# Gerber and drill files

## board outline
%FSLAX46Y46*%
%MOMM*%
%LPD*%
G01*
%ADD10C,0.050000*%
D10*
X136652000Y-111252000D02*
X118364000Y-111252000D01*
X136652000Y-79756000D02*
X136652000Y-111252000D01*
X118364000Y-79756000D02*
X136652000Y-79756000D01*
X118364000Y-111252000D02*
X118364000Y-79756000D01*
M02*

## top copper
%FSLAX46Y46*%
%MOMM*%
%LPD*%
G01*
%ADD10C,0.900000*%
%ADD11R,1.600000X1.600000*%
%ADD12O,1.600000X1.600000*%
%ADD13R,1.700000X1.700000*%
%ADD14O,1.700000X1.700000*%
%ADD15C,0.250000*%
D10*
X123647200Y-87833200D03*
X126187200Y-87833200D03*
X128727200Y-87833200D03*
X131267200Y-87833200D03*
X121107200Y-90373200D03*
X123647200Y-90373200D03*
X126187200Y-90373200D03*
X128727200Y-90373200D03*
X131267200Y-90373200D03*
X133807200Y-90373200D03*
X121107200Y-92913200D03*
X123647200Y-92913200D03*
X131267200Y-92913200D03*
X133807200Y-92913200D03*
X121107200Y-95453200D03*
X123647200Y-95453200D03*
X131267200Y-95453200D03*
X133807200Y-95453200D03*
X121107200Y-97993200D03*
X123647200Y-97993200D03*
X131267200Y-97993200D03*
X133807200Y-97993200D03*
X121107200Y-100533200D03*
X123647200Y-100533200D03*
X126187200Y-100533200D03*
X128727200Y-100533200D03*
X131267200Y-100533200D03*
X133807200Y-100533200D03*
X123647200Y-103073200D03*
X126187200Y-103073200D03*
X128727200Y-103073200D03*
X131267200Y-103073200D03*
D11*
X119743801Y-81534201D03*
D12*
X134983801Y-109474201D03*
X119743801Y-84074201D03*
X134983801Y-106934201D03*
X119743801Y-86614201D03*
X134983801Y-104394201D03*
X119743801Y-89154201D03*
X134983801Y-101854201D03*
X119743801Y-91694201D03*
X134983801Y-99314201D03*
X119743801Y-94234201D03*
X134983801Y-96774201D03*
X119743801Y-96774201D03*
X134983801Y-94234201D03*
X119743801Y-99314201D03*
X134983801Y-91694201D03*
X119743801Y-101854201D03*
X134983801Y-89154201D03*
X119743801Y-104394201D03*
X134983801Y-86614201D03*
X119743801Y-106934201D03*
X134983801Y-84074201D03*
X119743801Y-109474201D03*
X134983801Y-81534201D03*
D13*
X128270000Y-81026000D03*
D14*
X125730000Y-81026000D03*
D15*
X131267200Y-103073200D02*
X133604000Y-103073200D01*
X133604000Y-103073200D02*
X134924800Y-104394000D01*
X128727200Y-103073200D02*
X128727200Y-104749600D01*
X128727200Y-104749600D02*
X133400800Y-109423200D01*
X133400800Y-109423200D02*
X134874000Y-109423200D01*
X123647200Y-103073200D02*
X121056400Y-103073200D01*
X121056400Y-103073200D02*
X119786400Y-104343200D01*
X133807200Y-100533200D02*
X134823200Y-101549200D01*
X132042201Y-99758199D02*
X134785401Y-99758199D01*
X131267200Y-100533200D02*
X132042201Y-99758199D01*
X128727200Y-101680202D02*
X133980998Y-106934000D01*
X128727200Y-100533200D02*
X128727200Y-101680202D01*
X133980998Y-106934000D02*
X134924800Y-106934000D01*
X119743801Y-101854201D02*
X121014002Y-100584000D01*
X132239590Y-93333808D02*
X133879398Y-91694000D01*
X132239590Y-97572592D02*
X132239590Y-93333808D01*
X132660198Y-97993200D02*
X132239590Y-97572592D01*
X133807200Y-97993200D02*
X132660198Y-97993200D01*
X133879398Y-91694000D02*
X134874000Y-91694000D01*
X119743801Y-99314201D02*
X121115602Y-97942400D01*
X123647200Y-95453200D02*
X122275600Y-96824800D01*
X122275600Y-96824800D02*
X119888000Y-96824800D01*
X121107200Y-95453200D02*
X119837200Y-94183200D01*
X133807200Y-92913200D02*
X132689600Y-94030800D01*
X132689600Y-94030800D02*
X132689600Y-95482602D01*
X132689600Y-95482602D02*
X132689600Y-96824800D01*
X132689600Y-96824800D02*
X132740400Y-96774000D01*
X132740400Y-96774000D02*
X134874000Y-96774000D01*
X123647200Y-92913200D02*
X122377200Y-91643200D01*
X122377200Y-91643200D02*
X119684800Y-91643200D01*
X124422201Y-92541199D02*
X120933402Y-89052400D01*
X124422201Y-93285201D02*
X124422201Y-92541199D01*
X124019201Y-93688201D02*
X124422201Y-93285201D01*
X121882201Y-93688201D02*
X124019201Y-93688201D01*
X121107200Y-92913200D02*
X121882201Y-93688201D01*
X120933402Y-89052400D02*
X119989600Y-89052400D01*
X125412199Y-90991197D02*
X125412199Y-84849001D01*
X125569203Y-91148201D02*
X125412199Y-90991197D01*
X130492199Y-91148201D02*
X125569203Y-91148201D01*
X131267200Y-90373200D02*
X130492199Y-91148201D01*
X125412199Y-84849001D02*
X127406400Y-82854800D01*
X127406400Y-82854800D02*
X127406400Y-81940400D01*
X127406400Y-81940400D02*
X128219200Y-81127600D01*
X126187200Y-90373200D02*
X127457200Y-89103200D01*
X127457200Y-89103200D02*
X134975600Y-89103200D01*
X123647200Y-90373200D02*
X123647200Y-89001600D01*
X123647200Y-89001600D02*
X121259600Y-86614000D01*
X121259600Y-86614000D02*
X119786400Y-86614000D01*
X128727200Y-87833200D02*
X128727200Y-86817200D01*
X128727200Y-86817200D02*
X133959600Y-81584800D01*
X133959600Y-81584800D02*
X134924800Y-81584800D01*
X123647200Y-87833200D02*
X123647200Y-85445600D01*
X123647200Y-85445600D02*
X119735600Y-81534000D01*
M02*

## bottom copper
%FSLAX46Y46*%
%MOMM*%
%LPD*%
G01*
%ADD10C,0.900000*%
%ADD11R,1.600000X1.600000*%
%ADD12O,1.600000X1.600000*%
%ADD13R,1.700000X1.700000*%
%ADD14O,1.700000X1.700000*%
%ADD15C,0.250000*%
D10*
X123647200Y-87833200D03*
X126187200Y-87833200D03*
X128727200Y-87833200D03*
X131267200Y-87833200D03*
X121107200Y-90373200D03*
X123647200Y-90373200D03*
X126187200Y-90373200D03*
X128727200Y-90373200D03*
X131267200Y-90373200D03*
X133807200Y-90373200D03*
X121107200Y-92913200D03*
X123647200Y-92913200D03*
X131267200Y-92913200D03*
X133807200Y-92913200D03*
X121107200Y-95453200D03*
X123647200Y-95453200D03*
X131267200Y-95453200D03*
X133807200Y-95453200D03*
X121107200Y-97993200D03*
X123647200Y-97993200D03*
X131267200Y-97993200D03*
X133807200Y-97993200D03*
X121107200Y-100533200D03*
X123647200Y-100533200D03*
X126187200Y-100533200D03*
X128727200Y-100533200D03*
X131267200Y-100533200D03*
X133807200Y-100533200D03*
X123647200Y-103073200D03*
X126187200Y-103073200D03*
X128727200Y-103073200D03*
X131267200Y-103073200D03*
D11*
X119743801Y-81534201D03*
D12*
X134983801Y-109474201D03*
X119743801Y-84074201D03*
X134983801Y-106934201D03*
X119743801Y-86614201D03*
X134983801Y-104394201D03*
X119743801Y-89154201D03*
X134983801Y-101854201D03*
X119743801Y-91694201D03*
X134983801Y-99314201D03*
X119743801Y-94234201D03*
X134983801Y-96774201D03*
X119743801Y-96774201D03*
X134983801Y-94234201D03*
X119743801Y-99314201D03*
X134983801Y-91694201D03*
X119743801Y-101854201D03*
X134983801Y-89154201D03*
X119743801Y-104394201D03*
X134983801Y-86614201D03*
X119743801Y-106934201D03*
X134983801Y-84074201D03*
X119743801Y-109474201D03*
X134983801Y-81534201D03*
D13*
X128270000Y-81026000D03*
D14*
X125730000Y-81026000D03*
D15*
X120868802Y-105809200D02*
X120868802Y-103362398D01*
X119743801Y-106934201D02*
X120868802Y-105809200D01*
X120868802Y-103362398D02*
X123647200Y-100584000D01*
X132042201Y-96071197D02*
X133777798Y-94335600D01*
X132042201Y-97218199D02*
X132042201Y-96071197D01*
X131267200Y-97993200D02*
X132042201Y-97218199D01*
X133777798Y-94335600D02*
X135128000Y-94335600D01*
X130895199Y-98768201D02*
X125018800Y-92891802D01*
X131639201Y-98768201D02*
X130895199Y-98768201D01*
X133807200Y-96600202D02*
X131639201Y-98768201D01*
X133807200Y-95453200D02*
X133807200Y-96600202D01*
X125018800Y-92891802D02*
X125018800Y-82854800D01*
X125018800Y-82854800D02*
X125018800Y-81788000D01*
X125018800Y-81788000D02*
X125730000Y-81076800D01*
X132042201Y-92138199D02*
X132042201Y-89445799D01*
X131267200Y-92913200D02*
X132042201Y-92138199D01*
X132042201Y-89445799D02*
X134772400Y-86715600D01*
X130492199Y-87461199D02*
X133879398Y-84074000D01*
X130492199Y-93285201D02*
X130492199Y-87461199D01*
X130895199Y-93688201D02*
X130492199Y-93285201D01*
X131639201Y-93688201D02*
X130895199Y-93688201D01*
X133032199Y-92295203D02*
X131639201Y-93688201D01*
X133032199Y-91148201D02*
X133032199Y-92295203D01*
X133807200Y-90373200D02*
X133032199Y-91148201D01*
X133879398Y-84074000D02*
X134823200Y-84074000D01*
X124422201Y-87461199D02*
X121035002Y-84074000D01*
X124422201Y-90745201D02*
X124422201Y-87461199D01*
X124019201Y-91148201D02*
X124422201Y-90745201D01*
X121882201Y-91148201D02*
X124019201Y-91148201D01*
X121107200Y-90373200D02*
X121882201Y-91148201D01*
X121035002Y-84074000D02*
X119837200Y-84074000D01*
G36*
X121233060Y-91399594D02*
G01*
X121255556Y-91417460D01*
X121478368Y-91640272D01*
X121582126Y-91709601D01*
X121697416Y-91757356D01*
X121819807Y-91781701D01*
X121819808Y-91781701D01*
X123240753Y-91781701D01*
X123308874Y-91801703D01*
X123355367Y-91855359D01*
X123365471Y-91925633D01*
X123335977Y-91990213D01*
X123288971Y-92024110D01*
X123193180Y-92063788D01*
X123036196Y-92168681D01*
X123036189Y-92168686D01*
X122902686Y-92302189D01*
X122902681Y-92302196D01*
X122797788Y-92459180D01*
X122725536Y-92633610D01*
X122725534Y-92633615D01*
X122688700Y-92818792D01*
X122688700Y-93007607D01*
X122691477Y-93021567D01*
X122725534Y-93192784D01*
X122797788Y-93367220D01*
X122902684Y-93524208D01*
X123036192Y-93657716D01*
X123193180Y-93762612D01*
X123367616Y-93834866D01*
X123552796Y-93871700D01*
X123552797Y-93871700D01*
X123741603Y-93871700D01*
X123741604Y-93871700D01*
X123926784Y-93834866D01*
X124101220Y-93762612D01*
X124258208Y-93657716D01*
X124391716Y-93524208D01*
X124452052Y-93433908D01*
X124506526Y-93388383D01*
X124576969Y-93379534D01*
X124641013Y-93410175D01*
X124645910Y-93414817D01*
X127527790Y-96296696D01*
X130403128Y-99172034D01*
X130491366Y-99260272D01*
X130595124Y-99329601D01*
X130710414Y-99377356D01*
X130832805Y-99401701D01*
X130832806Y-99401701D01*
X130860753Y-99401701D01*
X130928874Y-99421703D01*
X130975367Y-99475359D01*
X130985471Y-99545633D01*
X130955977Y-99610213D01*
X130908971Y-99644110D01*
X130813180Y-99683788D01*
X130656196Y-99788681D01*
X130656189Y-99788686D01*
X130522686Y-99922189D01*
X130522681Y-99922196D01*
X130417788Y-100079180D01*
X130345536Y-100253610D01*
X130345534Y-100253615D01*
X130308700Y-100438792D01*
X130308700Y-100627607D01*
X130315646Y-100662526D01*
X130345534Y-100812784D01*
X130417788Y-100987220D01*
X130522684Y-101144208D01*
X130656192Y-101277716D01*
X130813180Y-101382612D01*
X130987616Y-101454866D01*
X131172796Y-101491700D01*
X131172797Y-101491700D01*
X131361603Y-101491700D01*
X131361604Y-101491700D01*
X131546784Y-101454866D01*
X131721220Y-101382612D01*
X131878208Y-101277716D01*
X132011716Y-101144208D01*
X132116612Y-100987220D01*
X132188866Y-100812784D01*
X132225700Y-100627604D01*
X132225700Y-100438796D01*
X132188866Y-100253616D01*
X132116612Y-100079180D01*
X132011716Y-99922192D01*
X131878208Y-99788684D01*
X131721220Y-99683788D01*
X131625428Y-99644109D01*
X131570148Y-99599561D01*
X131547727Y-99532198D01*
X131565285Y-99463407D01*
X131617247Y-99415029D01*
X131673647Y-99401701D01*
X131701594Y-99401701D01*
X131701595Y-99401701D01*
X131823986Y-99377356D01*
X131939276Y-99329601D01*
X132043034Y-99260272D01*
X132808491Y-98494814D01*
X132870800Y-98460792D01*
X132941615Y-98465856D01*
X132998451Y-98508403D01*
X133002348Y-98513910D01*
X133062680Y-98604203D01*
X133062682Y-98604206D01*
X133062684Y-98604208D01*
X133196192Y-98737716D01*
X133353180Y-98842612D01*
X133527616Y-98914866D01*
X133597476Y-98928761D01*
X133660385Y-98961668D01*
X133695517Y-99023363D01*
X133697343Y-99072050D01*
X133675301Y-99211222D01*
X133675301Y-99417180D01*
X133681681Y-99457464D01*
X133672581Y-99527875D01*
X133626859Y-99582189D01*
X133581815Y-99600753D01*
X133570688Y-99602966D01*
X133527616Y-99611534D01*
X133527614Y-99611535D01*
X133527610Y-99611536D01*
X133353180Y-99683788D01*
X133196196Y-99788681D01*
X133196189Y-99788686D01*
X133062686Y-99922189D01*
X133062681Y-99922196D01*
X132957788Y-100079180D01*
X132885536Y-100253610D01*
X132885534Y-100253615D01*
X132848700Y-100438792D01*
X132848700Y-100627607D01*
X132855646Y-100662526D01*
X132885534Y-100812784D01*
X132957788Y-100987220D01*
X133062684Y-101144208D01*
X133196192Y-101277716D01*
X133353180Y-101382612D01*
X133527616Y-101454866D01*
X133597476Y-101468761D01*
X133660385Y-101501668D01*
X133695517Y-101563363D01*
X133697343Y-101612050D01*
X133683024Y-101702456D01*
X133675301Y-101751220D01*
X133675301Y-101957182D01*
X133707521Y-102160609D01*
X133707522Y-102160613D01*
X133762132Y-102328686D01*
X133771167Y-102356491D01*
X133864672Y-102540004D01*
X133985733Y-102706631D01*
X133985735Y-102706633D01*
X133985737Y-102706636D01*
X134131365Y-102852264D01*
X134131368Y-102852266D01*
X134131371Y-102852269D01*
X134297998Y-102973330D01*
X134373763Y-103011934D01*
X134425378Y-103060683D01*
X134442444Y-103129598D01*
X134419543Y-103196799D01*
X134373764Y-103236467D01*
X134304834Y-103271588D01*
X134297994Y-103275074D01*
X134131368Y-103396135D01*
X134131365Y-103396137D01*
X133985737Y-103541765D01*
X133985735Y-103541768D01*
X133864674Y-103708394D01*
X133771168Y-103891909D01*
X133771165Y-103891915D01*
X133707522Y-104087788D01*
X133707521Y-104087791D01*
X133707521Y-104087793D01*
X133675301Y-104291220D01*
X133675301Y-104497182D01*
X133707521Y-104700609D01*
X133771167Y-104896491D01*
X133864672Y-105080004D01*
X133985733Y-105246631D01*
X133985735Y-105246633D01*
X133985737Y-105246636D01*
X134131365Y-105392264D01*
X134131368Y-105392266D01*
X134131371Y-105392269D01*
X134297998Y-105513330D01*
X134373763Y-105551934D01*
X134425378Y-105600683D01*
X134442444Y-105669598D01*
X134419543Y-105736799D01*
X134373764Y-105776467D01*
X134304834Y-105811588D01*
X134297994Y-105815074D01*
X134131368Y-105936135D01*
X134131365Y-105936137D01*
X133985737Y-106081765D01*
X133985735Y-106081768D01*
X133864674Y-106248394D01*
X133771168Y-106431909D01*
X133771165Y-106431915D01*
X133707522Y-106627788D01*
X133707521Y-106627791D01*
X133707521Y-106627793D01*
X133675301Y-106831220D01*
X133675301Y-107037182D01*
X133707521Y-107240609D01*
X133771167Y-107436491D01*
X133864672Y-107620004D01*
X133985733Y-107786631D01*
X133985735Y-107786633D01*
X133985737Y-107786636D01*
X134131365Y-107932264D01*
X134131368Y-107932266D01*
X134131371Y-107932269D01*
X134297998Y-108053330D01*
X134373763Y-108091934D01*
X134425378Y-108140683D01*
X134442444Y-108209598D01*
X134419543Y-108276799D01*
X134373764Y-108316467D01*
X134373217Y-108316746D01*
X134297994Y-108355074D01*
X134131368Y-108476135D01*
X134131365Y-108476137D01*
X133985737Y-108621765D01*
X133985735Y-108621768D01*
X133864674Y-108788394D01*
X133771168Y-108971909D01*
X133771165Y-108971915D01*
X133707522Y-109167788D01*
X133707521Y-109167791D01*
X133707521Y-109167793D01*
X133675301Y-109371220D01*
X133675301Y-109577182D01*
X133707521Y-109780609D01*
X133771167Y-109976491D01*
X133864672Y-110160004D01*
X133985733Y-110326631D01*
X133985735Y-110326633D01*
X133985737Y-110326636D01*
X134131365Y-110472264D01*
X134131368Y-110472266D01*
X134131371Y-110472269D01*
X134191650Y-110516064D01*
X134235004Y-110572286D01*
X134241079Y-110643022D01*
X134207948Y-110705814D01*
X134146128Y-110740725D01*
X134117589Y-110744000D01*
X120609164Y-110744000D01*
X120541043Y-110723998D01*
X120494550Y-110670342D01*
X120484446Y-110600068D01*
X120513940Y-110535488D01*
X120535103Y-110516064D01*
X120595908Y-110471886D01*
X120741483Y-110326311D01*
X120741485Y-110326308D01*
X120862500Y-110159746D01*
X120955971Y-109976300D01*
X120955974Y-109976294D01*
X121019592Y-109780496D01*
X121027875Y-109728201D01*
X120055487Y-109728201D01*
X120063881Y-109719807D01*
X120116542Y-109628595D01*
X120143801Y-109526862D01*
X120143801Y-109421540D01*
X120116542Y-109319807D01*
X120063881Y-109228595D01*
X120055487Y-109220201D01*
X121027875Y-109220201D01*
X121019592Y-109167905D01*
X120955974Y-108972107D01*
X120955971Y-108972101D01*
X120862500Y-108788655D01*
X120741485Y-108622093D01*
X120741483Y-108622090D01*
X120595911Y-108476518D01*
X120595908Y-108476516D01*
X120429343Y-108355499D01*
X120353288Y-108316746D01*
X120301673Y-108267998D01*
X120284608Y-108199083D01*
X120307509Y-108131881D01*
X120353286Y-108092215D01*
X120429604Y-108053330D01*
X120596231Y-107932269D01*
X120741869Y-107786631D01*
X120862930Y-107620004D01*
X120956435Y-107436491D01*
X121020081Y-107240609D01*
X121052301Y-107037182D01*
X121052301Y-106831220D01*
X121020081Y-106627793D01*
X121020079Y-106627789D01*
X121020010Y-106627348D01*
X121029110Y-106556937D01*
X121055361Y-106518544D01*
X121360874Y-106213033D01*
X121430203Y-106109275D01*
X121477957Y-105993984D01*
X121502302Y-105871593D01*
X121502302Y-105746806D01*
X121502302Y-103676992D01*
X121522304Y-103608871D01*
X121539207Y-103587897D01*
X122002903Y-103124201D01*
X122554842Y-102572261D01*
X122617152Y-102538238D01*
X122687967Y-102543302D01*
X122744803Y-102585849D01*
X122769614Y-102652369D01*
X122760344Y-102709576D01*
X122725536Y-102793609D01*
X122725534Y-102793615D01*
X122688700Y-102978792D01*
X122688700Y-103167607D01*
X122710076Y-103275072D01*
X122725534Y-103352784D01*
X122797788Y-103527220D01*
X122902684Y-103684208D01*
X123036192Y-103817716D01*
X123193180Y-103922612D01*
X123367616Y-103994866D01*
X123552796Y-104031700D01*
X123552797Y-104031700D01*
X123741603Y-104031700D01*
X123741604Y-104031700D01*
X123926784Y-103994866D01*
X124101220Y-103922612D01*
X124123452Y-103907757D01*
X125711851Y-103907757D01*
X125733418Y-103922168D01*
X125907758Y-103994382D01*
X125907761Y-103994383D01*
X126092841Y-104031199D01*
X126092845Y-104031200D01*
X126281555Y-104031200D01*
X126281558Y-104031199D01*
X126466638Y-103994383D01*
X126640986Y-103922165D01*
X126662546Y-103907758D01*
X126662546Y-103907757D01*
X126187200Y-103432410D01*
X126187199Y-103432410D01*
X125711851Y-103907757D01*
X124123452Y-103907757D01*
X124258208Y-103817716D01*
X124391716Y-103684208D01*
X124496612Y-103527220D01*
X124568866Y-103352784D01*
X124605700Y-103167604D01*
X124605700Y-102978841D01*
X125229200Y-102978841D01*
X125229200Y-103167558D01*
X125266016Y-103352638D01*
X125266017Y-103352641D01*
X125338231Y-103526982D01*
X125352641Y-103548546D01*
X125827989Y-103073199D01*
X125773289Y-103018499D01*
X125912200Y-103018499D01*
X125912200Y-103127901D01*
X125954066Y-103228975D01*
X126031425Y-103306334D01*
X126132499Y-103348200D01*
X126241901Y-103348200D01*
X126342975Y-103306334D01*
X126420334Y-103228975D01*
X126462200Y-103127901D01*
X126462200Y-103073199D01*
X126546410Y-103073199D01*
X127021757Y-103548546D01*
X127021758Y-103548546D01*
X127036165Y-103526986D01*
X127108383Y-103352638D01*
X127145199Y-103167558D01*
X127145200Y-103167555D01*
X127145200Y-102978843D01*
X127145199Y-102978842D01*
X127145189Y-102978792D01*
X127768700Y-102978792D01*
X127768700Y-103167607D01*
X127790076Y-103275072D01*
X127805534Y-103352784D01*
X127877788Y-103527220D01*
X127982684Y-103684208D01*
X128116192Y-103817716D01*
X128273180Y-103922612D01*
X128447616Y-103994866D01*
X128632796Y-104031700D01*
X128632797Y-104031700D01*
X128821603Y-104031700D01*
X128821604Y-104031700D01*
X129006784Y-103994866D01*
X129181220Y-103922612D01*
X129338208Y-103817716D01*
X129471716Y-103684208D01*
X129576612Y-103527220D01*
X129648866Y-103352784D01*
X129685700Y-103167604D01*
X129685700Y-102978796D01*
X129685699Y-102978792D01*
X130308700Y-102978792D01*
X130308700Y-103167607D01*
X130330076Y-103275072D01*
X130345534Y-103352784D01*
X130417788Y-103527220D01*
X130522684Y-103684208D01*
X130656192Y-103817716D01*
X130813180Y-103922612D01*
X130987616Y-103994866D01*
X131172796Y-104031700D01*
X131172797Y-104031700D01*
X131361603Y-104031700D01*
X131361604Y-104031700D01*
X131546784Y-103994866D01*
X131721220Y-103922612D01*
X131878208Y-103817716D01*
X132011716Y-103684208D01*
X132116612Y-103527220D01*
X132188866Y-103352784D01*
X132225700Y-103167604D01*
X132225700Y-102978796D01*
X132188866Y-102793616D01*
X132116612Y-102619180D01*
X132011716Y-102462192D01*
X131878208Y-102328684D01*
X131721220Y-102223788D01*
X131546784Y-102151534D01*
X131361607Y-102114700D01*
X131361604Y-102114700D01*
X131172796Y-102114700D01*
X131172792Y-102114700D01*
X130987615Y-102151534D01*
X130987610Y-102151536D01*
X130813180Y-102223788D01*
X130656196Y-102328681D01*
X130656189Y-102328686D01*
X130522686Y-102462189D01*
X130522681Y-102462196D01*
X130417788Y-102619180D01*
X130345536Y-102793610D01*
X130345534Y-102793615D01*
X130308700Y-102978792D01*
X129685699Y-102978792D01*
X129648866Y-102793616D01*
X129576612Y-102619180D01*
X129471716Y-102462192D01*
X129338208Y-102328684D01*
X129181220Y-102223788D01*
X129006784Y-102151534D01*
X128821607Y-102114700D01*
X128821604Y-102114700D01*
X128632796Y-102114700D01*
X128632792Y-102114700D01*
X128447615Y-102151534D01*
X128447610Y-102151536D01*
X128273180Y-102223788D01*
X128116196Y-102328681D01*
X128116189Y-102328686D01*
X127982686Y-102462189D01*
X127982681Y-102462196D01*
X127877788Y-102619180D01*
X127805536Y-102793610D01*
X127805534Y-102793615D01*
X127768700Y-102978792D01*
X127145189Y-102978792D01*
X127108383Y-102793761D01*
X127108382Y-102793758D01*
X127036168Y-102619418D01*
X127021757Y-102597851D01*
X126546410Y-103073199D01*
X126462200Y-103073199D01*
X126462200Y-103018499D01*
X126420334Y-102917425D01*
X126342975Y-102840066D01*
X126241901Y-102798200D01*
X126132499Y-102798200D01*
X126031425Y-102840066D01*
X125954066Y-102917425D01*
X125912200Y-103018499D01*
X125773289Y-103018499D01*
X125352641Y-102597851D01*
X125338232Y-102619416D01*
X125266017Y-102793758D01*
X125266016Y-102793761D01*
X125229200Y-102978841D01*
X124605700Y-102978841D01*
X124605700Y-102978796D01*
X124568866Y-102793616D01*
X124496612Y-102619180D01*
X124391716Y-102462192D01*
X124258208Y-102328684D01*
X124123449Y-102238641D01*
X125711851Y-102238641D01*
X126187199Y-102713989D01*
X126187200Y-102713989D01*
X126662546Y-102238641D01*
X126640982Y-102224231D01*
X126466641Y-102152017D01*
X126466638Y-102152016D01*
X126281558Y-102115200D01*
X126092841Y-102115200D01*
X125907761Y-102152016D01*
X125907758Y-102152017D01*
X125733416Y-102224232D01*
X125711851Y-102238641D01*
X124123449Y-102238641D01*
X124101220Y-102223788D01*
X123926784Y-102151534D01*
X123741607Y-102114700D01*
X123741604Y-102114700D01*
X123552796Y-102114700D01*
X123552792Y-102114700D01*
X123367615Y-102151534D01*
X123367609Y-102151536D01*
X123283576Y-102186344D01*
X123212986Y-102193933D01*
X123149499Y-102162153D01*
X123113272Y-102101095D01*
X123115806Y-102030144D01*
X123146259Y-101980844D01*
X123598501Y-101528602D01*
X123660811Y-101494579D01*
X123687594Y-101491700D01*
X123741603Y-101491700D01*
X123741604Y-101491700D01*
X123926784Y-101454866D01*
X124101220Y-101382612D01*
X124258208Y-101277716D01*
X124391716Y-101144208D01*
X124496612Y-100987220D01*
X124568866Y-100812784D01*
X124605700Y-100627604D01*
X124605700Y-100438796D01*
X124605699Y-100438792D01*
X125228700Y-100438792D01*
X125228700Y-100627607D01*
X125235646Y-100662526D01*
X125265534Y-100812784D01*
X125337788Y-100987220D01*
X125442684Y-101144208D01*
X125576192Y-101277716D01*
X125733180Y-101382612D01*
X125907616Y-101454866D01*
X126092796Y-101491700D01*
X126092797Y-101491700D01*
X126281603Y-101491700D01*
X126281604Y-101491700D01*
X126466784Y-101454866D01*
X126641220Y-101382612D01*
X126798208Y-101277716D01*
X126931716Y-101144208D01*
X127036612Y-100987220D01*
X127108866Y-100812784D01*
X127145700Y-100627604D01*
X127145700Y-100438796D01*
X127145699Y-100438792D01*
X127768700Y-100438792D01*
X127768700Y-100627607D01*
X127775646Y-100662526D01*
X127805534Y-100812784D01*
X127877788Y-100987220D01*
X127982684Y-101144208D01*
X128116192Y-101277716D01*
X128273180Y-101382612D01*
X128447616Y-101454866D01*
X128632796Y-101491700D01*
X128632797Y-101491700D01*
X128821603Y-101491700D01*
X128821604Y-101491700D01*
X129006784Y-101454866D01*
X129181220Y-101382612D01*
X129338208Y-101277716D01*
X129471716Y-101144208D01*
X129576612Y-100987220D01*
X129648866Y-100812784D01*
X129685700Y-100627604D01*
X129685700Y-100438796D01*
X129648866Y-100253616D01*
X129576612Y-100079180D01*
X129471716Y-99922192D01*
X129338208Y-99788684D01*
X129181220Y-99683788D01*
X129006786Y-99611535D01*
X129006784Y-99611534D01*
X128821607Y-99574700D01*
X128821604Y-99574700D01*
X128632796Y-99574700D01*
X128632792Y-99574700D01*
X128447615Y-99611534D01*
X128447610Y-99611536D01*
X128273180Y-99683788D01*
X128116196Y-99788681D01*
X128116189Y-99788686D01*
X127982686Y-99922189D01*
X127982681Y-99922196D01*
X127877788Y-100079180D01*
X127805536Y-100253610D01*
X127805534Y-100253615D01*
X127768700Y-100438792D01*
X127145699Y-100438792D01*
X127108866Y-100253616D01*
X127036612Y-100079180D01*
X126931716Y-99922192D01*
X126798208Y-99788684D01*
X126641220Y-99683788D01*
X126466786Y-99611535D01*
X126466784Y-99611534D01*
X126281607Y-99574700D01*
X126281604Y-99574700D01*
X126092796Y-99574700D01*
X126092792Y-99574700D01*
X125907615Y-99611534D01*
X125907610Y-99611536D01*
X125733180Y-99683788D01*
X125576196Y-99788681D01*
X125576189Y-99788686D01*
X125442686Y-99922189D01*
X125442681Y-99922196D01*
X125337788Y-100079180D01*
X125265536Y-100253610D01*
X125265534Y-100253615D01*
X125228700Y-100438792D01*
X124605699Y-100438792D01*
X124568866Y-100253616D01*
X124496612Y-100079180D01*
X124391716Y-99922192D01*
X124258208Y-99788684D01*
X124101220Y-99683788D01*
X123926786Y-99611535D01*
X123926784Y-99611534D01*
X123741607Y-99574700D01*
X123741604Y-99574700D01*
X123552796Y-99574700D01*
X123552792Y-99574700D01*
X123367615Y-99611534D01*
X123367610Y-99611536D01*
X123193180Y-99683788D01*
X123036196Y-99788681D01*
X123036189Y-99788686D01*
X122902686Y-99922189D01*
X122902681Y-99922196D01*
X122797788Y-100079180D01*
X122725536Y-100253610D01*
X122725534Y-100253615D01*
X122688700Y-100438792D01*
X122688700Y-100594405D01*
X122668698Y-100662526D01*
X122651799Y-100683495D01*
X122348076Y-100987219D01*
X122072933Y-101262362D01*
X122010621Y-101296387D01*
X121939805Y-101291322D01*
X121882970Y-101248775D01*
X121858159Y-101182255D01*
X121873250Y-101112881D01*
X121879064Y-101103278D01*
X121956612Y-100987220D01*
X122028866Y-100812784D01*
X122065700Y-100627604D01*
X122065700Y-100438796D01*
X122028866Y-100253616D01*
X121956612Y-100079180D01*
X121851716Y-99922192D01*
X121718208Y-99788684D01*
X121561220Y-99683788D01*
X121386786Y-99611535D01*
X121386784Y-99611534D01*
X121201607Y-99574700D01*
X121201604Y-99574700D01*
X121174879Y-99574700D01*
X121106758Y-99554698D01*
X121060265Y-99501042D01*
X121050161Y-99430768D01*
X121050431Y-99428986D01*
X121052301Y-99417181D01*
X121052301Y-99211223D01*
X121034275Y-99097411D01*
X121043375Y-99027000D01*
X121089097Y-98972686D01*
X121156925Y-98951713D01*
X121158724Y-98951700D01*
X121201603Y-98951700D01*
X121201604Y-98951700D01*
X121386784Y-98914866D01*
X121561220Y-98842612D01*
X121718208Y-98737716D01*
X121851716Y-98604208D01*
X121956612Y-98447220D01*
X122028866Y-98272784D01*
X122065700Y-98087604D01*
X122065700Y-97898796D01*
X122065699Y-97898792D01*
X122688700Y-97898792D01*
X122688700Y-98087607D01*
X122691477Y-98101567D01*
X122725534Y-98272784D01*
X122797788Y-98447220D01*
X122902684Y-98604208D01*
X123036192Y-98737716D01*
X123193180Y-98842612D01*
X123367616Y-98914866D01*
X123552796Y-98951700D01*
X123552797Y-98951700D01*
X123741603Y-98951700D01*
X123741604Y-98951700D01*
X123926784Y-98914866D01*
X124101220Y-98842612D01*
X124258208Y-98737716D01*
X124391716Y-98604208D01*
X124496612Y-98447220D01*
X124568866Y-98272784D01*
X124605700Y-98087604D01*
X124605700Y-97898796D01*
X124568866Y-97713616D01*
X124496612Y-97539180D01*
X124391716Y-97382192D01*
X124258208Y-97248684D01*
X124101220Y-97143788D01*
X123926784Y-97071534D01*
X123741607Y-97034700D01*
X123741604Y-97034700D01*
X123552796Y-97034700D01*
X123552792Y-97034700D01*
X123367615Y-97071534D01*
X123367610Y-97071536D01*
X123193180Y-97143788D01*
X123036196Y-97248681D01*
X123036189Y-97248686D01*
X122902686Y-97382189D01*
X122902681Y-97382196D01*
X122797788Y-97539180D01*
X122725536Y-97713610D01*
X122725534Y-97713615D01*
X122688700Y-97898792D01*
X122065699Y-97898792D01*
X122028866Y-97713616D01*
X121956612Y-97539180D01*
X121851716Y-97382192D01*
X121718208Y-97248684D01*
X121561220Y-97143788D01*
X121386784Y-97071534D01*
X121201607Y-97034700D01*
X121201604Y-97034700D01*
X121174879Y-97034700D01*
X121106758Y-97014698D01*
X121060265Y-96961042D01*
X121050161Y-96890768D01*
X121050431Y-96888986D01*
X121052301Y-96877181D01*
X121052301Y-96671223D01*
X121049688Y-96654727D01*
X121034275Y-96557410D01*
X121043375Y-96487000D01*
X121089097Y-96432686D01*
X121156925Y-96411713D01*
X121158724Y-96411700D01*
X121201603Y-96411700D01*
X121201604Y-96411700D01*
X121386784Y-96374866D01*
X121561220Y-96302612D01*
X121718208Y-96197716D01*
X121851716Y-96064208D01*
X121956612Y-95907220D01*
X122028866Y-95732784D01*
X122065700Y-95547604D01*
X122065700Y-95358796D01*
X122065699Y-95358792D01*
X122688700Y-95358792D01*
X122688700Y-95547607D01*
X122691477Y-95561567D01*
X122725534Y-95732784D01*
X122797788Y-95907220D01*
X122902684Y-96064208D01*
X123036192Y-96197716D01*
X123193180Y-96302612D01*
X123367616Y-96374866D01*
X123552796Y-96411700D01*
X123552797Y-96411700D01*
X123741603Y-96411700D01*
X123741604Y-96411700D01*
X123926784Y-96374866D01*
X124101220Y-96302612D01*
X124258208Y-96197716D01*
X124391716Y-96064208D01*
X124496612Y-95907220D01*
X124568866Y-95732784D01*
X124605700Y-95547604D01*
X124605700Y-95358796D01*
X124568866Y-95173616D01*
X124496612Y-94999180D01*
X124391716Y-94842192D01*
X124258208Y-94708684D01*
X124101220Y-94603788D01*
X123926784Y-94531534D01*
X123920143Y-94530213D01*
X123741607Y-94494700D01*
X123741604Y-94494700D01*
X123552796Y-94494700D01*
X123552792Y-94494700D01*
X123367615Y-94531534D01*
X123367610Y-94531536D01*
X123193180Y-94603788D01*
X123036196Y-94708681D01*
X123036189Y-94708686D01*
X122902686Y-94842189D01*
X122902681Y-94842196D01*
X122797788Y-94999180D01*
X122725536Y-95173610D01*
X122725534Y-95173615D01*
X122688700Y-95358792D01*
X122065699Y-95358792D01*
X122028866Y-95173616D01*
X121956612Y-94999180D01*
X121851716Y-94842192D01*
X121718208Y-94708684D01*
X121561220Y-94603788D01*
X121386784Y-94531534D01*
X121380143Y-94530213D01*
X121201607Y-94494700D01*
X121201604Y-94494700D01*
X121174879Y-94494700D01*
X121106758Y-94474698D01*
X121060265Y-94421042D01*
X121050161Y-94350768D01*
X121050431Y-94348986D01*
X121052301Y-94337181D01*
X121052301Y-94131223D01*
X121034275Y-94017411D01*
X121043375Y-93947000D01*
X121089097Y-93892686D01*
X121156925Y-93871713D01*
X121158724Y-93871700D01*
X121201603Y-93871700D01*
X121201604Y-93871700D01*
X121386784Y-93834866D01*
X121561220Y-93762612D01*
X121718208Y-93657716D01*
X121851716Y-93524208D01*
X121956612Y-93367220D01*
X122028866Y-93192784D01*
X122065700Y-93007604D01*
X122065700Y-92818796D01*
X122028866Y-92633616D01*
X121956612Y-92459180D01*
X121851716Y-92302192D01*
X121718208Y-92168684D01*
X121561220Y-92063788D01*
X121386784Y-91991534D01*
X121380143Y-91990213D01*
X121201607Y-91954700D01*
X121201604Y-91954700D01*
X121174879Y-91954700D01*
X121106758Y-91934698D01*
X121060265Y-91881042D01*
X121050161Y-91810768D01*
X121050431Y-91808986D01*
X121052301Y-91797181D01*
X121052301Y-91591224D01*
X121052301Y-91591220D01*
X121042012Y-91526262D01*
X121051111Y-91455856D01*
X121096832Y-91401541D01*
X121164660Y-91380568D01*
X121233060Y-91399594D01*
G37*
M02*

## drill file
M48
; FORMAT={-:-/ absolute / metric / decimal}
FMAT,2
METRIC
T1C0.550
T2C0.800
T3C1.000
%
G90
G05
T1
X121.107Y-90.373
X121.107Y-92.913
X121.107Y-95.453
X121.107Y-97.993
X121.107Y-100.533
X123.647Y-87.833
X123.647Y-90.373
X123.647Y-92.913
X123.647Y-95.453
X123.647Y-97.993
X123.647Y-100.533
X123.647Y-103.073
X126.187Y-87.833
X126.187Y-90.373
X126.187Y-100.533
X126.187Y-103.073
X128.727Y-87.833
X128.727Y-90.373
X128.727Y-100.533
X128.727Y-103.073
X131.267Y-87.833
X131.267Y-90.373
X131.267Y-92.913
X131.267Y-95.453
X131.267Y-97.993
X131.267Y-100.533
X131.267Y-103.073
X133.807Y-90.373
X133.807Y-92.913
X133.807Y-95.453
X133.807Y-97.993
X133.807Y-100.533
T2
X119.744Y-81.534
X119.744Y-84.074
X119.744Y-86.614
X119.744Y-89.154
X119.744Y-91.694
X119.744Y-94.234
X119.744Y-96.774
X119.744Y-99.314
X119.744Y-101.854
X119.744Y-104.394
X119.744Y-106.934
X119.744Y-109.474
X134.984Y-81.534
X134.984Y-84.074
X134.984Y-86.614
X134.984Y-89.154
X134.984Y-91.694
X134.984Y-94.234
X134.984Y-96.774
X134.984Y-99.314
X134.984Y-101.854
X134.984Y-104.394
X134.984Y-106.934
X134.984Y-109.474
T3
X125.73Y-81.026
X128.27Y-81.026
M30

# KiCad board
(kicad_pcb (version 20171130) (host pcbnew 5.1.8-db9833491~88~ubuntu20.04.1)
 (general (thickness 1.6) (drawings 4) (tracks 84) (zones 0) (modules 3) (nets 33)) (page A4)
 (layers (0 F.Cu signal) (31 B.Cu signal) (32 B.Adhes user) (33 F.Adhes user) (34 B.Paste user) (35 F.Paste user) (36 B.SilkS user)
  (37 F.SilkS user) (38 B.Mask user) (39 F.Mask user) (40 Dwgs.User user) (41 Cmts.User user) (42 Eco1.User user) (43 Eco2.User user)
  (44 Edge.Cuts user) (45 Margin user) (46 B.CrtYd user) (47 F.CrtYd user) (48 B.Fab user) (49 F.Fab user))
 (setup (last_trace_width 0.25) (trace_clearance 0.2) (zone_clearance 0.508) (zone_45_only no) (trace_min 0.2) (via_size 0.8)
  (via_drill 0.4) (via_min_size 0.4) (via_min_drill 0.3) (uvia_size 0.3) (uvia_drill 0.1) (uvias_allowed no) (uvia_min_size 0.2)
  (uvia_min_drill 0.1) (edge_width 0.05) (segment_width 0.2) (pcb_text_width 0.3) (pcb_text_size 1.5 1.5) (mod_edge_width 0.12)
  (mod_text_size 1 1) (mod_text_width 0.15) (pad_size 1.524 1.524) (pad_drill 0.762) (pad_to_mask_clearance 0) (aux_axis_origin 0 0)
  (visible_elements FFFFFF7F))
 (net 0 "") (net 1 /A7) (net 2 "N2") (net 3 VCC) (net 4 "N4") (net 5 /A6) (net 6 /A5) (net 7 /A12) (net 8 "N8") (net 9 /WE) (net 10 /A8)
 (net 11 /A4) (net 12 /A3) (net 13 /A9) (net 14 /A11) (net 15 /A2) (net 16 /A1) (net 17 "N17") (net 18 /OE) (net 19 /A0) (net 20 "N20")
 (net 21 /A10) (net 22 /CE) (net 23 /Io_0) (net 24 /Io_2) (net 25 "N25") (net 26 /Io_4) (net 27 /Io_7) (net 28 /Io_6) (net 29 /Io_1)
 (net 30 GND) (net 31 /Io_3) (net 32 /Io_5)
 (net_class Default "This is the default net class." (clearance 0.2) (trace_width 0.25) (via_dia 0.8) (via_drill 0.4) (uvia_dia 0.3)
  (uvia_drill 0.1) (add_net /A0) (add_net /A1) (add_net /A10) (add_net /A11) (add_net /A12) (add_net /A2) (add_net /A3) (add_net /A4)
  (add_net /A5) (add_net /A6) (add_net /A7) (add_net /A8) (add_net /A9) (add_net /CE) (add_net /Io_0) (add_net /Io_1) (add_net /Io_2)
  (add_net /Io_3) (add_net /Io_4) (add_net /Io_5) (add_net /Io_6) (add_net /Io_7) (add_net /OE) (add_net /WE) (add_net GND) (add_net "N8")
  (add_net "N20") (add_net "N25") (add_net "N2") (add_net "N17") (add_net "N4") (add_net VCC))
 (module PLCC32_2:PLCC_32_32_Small (layer F.Cu) (at 127.4572 95.4532)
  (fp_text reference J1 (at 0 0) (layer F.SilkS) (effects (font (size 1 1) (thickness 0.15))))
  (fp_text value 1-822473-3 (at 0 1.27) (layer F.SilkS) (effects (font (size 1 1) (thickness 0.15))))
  (pad 4 thru_hole circle (at -3.81 -7.62) (size 0.9 0.9) (drill 0.55) (layers *.Cu *.Mask) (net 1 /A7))
  (pad 2 thru_hole circle (at -1.27 -7.62) (size 0.9 0.9) (drill 0.55) (layers *.Cu *.Mask) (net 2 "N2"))
  (pad 32 thru_hole circle (at 1.27 -7.62) (size 0.9 0.9) (drill 0.55) (layers *.Cu *.Mask) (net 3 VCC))
  (pad 30 thru_hole circle (at 3.81 -7.62) (size 0.9 0.9) (drill 0.55) (layers *.Cu *.Mask) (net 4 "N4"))
  (pad 5 thru_hole circle (at -6.35 -5.08) (size 0.9 0.9) (drill 0.55) (layers *.Cu *.Mask) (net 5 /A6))
  (pad 6 thru_hole circle (at -3.81 -5.08) (size 0.9 0.9) (drill 0.55) (layers *.Cu *.Mask) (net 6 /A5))
  (pad 3 thru_hole circle (at -1.27 -5.08) (size 0.9 0.9) (drill 0.55) (layers *.Cu *.Mask) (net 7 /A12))
  (pad 1 thru_hole circle (at 1.27 -5.08) (size 0.9 0.9) (drill 0.55) (layers *.Cu *.Mask) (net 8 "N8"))
  (pad 31 thru_hole circle (at 3.81 -5.08) (size 0.9 0.9) (drill 0.55) (layers *.Cu *.Mask) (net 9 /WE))
  (pad 29 thru_hole circle (at 6.35 -5.08) (size 0.9 0.9) (drill 0.55) (layers *.Cu *.Mask) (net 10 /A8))
  (pad 7 thru_hole circle (at -6.35 -2.54) (size 0.9 0.9) (drill 0.55) (layers *.Cu *.Mask) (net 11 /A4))
  (pad 8 thru_hole circle (at -3.81 -2.54) (size 0.9 0.9) (drill 0.55) (layers *.Cu *.Mask) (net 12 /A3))
  (pad 28 thru_hole circle (at 3.81 -2.54) (size 0.9 0.9) (drill 0.55) (layers *.Cu *.Mask) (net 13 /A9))
  (pad 27 thru_hole circle (at 6.35 -2.54) (size 0.9 0.9) (drill 0.55) (layers *.Cu *.Mask) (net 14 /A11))
  (pad 9 thru_hole circle (at -6.35 0) (size 0.9 0.9) (drill 0.55) (layers *.Cu *.Mask) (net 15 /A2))
  (pad 10 thru_hole circle (at -3.81 0) (size 0.9 0.9) (drill 0.55) (layers *.Cu *.Mask) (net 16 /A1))
  (pad 26 thru_hole circle (at 3.81 0) (size 0.9 0.9) (drill 0.55) (layers *.Cu *.Mask) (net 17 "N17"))
  (pad 25 thru_hole circle (at 6.35 0) (size 0.9 0.9) (drill 0.55) (layers *.Cu *.Mask) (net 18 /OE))
  (pad 11 thru_hole circle (at -6.35 2.54) (size 0.9 0.9) (drill 0.55) (layers *.Cu *.Mask) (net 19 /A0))
  (pad 12 thru_hole circle (at -3.81 2.54) (size 0.9 0.9) (drill 0.55) (layers *.Cu *.Mask) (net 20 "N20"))
  (pad 24 thru_hole circle (at 3.81 2.54) (size 0.9 0.9) (drill 0.55) (layers *.Cu *.Mask) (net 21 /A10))
  (pad 23 thru_hole circle (at 6.35 2.54) (size 0.9 0.9) (drill 0.55) (layers *.Cu *.Mask) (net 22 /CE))
  (pad 13 thru_hole circle (at -6.35 5.08) (size 0.9 0.9) (drill 0.55) (layers *.Cu *.Mask) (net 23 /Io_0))
  (pad 15 thru_hole circle (at -3.81 5.08) (size 0.9 0.9) (drill 0.55) (layers *.Cu *.Mask) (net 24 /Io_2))
  (pad 17 thru_hole circle (at -1.27 5.08) (size 0.9 0.9) (drill 0.55) (layers *.Cu *.Mask) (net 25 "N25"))
  (pad 19 thru_hole circle (at 1.27 5.08) (size 0.9 0.9) (drill 0.55) (layers *.Cu *.Mask) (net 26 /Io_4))
  (pad 22 thru_hole circle (at 3.81 5.08) (size 0.9 0.9) (drill 0.55) (layers *.Cu *.Mask) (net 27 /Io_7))
  (pad 21 thru_hole circle (at 6.35 5.08) (size 0.9 0.9) (drill 0.55) (layers *.Cu *.Mask) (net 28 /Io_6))
  (pad 14 thru_hole circle (at -3.81 7.62) (size 0.9 0.9) (drill 0.55) (layers *.Cu *.Mask) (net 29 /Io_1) (die_length 1))
  (pad 16 thru_hole circle (at -1.27 7.62) (size 0.9 0.9) (drill 0.55) (layers *.Cu *.Mask) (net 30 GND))
  (pad 18 thru_hole circle (at 1.27 7.62) (size 0.9 0.9) (drill 0.55) (layers *.Cu *.Mask) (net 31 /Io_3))
  (pad 20 thru_hole circle (at 3.81 7.62) (size 0.9 0.9) (drill 0.55) (layers *.Cu *.Mask) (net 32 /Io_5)))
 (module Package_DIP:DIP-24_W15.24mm (layer F.Cu) (at 119.743801 81.534201)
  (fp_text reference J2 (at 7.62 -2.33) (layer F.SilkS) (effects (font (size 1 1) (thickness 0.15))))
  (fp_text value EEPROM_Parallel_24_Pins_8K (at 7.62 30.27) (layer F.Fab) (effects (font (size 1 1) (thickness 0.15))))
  (pad 1 thru_hole rect (at 0 0) (size 1.6 1.6) (drill 0.8) (layers *.Cu *.Mask) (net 1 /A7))
  (pad 13 thru_hole oval (at 15.24 27.94) (size 1.6 1.6) (drill 0.8) (layers *.Cu *.Mask) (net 31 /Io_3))
  (pad 2 thru_hole oval (at 0 2.54) (size 1.6 1.6) (drill 0.8) (layers *.Cu *.Mask) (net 5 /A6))
  (pad 14 thru_hole oval (at 15.24 25.4) (size 1.6 1.6) (drill 0.8) (layers *.Cu *.Mask) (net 26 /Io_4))
  (pad 3 thru_hole oval (at 0 5.08) (size 1.6 1.6) (drill 0.8) (layers *.Cu *.Mask) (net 6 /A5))
  (pad 15 thru_hole oval (at 15.24 22.86) (size 1.6 1.6) (drill 0.8) (layers *.Cu *.Mask) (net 32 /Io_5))
  (pad 4 thru_hole oval (at 0 7.62) (size 1.6 1.6) (drill 0.8) (layers *.Cu *.Mask) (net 11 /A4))
  (pad 16 thru_hole oval (at 15.24 20.32) (size 1.6 1.6) (drill 0.8) (layers *.Cu *.Mask) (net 28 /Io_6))
  (pad 5 thru_hole oval (at 0 10.16) (size 1.6 1.6) (drill 0.8) (layers *.Cu *.Mask) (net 12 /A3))
  (pad 17 thru_hole oval (at 15.24 17.78) (size 1.6 1.6) (drill 0.8) (layers *.Cu *.Mask) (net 27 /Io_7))
  (pad 6 thru_hole oval (at 0 12.7) (size 1.6 1.6) (drill 0.8) (layers *.Cu *.Mask) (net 15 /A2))
  (pad 18 thru_hole oval (at 15.24 15.24) (size 1.6 1.6) (drill 0.8) (layers *.Cu *.Mask) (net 14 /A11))
  (pad 7 thru_hole oval (at 0 15.24) (size 1.6 1.6) (drill 0.8) (layers *.Cu *.Mask) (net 16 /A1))
  (pad 19 thru_hole oval (at 15.24 12.7) (size 1.6 1.6) (drill 0.8) (layers *.Cu *.Mask) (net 21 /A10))
  (pad 8 thru_hole oval (at 0 17.78) (size 1.6 1.6) (drill 0.8) (layers *.Cu *.Mask) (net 19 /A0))
  (pad 20 thru_hole oval (at 15.24 10.16) (size 1.6 1.6) (drill 0.8) (layers *.Cu *.Mask) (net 22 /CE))
  (pad 9 thru_hole oval (at 0 20.32) (size 1.6 1.6) (drill 0.8) (layers *.Cu *.Mask) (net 23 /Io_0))
  (pad 21 thru_hole oval (at 15.24 7.62) (size 1.6 1.6) (drill 0.8) (layers *.Cu *.Mask) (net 7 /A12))
  (pad 10 thru_hole oval (at 0 22.86) (size 1.6 1.6) (drill 0.8) (layers *.Cu *.Mask) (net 29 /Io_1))
  (pad 22 thru_hole oval (at 15.24 5.08) (size 1.6 1.6) (drill 0.8) (layers *.Cu *.Mask) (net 13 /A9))
  (pad 11 thru_hole oval (at 0 25.4) (size 1.6 1.6) (drill 0.8) (layers *.Cu *.Mask) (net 24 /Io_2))
  (pad 23 thru_hole oval (at 15.24 2.54) (size 1.6 1.6) (drill 0.8) (layers *.Cu *.Mask) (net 10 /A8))
  (pad 12 thru_hole oval (at 0 27.94) (size 1.6 1.6) (drill 0.8) (layers *.Cu *.Mask) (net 30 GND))
  (pad 24 thru_hole oval (at 15.24 0) (size 1.6 1.6) (drill 0.8) (layers *.Cu *.Mask) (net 3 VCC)))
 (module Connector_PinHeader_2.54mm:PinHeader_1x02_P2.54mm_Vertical (layer F.Cu) (at 128.27 81.026 270)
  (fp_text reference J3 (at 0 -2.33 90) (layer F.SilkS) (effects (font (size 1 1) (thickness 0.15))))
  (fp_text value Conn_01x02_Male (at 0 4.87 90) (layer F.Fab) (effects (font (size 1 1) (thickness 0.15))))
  (pad 1 thru_hole rect (at 0 0 270) (size 1.7 1.7) (drill 1) (layers *.Cu *.Mask) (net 9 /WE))
  (pad 2 thru_hole oval (at 0 2.54 270) (size 1.7 1.7) (drill 1) (layers *.Cu *.Mask) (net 18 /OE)))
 (gr_line (start 136.652 111.252) (end 118.364 111.252) (layer Edge.Cuts) (width 0.05))
 (gr_line (start 136.652 79.756) (end 136.652 111.252) (layer Edge.Cuts) (width 0.05))
 (gr_line (start 118.364 79.756) (end 136.652 79.756) (layer Edge.Cuts) (width 0.05))
 (gr_line (start 118.364 111.252) (end 118.364 79.756) (layer Edge.Cuts) (width 0.05))
 (segment (start 131.2672 103.0732) (end 133.604 103.0732) (width 0.25) (layer F.Cu) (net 32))
 (segment (start 133.604 103.0732) (end 134.9248 104.394) (width 0.25) (layer F.Cu) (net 32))
 (segment (start 128.7272 103.0732) (end 128.7272 104.7496) (width 0.25) (layer F.Cu) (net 31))
 (segment (start 128.7272 104.7496) (end 133.4008 109.4232) (width 0.25) (layer F.Cu) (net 31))
 (segment (start 133.4008 109.4232) (end 134.874 109.4232) (width 0.25) (layer F.Cu) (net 31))
 (segment (start 123.6472 103.0732) (end 121.0564 103.0732) (width 0.25) (layer F.Cu) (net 29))
 (segment (start 121.0564 103.0732) (end 119.7864 104.3432) (width 0.25) (layer F.Cu) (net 29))
 (segment (start 133.8072 100.5332) (end 134.8232 101.5492) (width 0.25) (layer F.Cu) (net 28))
 (segment (start 132.042201 99.758199) (end 134.785401 99.758199) (width 0.25) (layer F.Cu) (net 27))
 (segment (start 131.2672 100.5332) (end 132.042201 99.758199) (width 0.25) (layer F.Cu) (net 27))
 (segment (start 128.7272 101.680202) (end 133.980998 106.934) (width 0.25) (layer F.Cu) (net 26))
 (segment (start 128.7272 100.5332) (end 128.7272 101.680202) (width 0.25) (layer F.Cu) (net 26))
 (segment (start 133.980998 106.934) (end 134.9248 106.934) (width 0.25) (layer F.Cu) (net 26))
 (segment (start 120.868802 105.8092) (end 120.868802 103.362398) (width 0.25) (layer B.Cu) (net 24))
 (segment (start 119.743801 106.934201) (end 120.868802 105.8092) (width 0.25) (layer B.Cu) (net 24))
 (segment (start 120.868802 103.362398) (end 123.6472 100.584) (width 0.25) (layer B.Cu) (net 24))
 (segment (start 119.743801 101.854201) (end 121.014002 100.584) (width 0.25) (layer F.Cu) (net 23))
 (segment (start 132.23959 93.333808) (end 133.879398 91.694) (width 0.25) (layer F.Cu) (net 22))
 (segment (start 132.23959 97.572592) (end 132.23959 93.333808) (width 0.25) (layer F.Cu) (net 22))
 (segment (start 132.660198 97.9932) (end 132.23959 97.572592) (width 0.25) (layer F.Cu) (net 22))
 (segment (start 133.8072 97.9932) (end 132.660198 97.9932) (width 0.25) (layer F.Cu) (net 22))
 (segment (start 133.879398 91.694) (end 134.874 91.694) (width 0.25) (layer F.Cu) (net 22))
 (segment (start 132.042201 96.071197) (end 133.777798 94.3356) (width 0.25) (layer B.Cu) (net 21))
 (segment (start 132.042201 97.218199) (end 132.042201 96.071197) (width 0.25) (layer B.Cu) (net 21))
 (segment (start 131.2672 97.9932) (end 132.042201 97.218199) (width 0.25) (layer B.Cu) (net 21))
 (segment (start 133.777798 94.3356) (end 135.128 94.3356) (width 0.25) (layer B.Cu) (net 21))
 (segment (start 119.743801 99.314201) (end 121.115602 97.9424) (width 0.25) (layer F.Cu) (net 19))
 (segment (start 130.895199 98.768201) (end 125.0188 92.891802) (width 0.25) (layer B.Cu) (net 18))
 (segment (start 131.639201 98.768201) (end 130.895199 98.768201) (width 0.25) (layer B.Cu) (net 18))
 (segment (start 133.8072 96.600202) (end 131.639201 98.768201) (width 0.25) (layer B.Cu) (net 18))
 (segment (start 133.8072 95.4532) (end 133.8072 96.600202) (width 0.25) (layer B.Cu) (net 18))
 (segment (start 125.0188 92.891802) (end 125.0188 82.8548) (width 0.25) (layer B.Cu) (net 18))
 (segment (start 125.0188 82.8548) (end 125.0188 81.788) (width 0.25) (layer B.Cu) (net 18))
 (segment (start 125.0188 81.788) (end 125.73 81.0768) (width 0.25) (layer B.Cu) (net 18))
 (segment (start 123.6472 95.4532) (end 122.2756 96.8248) (width 0.25) (layer F.Cu) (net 16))
 (segment (start 122.2756 96.8248) (end 119.888 96.8248) (width 0.25) (layer F.Cu) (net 16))
 (segment (start 121.1072 95.4532) (end 119.8372 94.1832) (width 0.25) (layer F.Cu) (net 15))
 (segment (start 133.8072 92.9132) (end 132.6896 94.0308) (width 0.25) (layer F.Cu) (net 14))
 (segment (start 132.6896 94.0308) (end 132.6896 95.482602) (width 0.25) (layer F.Cu) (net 14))
 (segment (start 132.6896 95.482602) (end 132.6896 96.8248) (width 0.25) (layer F.Cu) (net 14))
 (segment (start 132.6896 96.8248) (end 132.7404 96.774) (width 0.25) (layer F.Cu) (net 14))
 (segment (start 132.7404 96.774) (end 134.874 96.774) (width 0.25) (layer F.Cu) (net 14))
 (segment (start 132.042201 92.138199) (end 132.042201 89.445799) (width 0.25) (layer B.Cu) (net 13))
 (segment (start 131.2672 92.9132) (end 132.042201 92.138199) (width 0.25) (layer B.Cu) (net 13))
 (segment (start 132.042201 89.445799) (end 134.7724 86.7156) (width 0.25) (layer B.Cu) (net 13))
 (segment (start 123.6472 92.9132) (end 122.3772 91.6432) (width 0.25) (layer F.Cu) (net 12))
 (segment (start 122.3772 91.6432) (end 119.6848 91.6432) (width 0.25) (layer F.Cu) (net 12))
 (segment (start 124.422201 92.541199) (end 120.933402 89.0524) (width 0.25) (layer F.Cu) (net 11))
 (segment (start 124.422201 93.285201) (end 124.422201 92.541199) (width 0.25) (layer F.Cu) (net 11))
 (segment (start 124.019201 93.688201) (end 124.422201 93.285201) (width 0.25) (layer F.Cu) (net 11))
 (segment (start 121.882201 93.688201) (end 124.019201 93.688201) (width 0.25) (layer F.Cu) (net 11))
 (segment (start 121.1072 92.9132) (end 121.882201 93.688201) (width 0.25) (layer F.Cu) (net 11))
 (segment (start 120.933402 89.0524) (end 119.9896 89.0524) (width 0.25) (layer F.Cu) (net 11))
 (segment (start 130.492199 87.461199) (end 133.879398 84.074) (width 0.25) (layer B.Cu) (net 10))
 (segment (start 130.492199 93.285201) (end 130.492199 87.461199) (width 0.25) (layer B.Cu) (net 10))
 (segment (start 130.895199 93.688201) (end 130.492199 93.285201) (width 0.25) (layer B.Cu) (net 10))
 (segment (start 131.639201 93.688201) (end 130.895199 93.688201) (width 0.25) (layer B.Cu) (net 10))
 (segment (start 133.032199 92.295203) (end 131.639201 93.688201) (width 0.25) (layer B.Cu) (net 10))
 (segment (start 133.032199 91.148201) (end 133.032199 92.295203) (width 0.25) (layer B.Cu) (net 10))
 (segment (start 133.8072 90.3732) (end 133.032199 91.148201) (width 0.25) (layer B.Cu) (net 10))
 (segment (start 133.879398 84.074) (end 134.8232 84.074) (width 0.25) (layer B.Cu) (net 10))
 (segment (start 125.412199 90.991197) (end 125.412199 84.849001) (width 0.25) (layer F.Cu) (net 9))
 (segment (start 125.569203 91.148201) (end 125.412199 90.991197) (width 0.25) (layer F.Cu) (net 9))
 (segment (start 130.492199 91.148201) (end 125.569203 91.148201) (width 0.25) (layer F.Cu) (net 9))
 (segment (start 131.2672 90.3732) (end 130.492199 91.148201) (width 0.25) (layer F.Cu) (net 9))
 (segment (start 125.412199 84.849001) (end 127.4064 82.8548) (width 0.25) (layer F.Cu) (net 9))
 (segment (start 127.4064 82.8548) (end 127.4064 81.9404) (width 0.25) (layer F.Cu) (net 9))
 (segment (start 127.4064 81.9404) (end 128.2192 81.1276) (width 0.25) (layer F.Cu) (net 9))
 (segment (start 126.1872 90.3732) (end 127.4572 89.1032) (width 0.25) (layer F.Cu) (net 7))
 (segment (start 127.4572 89.1032) (end 134.9756 89.1032) (width 0.25) (layer F.Cu) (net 7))
 (segment (start 123.6472 90.3732) (end 123.6472 89.0016) (width 0.25) (layer F.Cu) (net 6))
 (segment (start 123.6472 89.0016) (end 121.2596 86.614) (width 0.25) (layer F.Cu) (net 6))
 (segment (start 121.2596 86.614) (end 119.7864 86.614) (width 0.25) (layer F.Cu) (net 6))
 (segment (start 124.422201 87.461199) (end 121.035002 84.074) (width 0.25) (layer B.Cu) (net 5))
 (segment (start 124.422201 90.745201) (end 124.422201 87.461199) (width 0.25) (layer B.Cu) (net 5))
 (segment (start 124.019201 91.148201) (end 124.422201 90.745201) (width 0.25) (layer B.Cu) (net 5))
 (segment (start 121.882201 91.148201) (end 124.019201 91.148201) (width 0.25) (layer B.Cu) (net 5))
 (segment (start 121.1072 90.3732) (end 121.882201 91.148201) (width 0.25) (layer B.Cu) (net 5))
 (segment (start 121.035002 84.074) (end 119.8372 84.074) (width 0.25) (layer B.Cu) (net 5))
 (segment (start 128.7272 87.8332) (end 128.7272 86.8172) (width 0.25) (layer F.Cu) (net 3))
 (segment (start 128.7272 86.8172) (end 133.9596 81.5848) (width 0.25) (layer F.Cu) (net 3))
 (segment (start 133.9596 81.5848) (end 134.9248 81.5848) (width 0.25) (layer F.Cu) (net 3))
 (segment (start 123.6472 87.8332) (end 123.6472 85.4456) (width 0.25) (layer F.Cu) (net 1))
 (segment (start 123.6472 85.4456) (end 119.7356 81.534) (width 0.25) (layer F.Cu) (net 1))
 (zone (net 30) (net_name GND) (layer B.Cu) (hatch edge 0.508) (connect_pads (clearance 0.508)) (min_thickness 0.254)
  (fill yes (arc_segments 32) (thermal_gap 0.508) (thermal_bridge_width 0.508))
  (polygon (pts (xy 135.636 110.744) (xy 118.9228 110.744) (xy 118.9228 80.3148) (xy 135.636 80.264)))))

